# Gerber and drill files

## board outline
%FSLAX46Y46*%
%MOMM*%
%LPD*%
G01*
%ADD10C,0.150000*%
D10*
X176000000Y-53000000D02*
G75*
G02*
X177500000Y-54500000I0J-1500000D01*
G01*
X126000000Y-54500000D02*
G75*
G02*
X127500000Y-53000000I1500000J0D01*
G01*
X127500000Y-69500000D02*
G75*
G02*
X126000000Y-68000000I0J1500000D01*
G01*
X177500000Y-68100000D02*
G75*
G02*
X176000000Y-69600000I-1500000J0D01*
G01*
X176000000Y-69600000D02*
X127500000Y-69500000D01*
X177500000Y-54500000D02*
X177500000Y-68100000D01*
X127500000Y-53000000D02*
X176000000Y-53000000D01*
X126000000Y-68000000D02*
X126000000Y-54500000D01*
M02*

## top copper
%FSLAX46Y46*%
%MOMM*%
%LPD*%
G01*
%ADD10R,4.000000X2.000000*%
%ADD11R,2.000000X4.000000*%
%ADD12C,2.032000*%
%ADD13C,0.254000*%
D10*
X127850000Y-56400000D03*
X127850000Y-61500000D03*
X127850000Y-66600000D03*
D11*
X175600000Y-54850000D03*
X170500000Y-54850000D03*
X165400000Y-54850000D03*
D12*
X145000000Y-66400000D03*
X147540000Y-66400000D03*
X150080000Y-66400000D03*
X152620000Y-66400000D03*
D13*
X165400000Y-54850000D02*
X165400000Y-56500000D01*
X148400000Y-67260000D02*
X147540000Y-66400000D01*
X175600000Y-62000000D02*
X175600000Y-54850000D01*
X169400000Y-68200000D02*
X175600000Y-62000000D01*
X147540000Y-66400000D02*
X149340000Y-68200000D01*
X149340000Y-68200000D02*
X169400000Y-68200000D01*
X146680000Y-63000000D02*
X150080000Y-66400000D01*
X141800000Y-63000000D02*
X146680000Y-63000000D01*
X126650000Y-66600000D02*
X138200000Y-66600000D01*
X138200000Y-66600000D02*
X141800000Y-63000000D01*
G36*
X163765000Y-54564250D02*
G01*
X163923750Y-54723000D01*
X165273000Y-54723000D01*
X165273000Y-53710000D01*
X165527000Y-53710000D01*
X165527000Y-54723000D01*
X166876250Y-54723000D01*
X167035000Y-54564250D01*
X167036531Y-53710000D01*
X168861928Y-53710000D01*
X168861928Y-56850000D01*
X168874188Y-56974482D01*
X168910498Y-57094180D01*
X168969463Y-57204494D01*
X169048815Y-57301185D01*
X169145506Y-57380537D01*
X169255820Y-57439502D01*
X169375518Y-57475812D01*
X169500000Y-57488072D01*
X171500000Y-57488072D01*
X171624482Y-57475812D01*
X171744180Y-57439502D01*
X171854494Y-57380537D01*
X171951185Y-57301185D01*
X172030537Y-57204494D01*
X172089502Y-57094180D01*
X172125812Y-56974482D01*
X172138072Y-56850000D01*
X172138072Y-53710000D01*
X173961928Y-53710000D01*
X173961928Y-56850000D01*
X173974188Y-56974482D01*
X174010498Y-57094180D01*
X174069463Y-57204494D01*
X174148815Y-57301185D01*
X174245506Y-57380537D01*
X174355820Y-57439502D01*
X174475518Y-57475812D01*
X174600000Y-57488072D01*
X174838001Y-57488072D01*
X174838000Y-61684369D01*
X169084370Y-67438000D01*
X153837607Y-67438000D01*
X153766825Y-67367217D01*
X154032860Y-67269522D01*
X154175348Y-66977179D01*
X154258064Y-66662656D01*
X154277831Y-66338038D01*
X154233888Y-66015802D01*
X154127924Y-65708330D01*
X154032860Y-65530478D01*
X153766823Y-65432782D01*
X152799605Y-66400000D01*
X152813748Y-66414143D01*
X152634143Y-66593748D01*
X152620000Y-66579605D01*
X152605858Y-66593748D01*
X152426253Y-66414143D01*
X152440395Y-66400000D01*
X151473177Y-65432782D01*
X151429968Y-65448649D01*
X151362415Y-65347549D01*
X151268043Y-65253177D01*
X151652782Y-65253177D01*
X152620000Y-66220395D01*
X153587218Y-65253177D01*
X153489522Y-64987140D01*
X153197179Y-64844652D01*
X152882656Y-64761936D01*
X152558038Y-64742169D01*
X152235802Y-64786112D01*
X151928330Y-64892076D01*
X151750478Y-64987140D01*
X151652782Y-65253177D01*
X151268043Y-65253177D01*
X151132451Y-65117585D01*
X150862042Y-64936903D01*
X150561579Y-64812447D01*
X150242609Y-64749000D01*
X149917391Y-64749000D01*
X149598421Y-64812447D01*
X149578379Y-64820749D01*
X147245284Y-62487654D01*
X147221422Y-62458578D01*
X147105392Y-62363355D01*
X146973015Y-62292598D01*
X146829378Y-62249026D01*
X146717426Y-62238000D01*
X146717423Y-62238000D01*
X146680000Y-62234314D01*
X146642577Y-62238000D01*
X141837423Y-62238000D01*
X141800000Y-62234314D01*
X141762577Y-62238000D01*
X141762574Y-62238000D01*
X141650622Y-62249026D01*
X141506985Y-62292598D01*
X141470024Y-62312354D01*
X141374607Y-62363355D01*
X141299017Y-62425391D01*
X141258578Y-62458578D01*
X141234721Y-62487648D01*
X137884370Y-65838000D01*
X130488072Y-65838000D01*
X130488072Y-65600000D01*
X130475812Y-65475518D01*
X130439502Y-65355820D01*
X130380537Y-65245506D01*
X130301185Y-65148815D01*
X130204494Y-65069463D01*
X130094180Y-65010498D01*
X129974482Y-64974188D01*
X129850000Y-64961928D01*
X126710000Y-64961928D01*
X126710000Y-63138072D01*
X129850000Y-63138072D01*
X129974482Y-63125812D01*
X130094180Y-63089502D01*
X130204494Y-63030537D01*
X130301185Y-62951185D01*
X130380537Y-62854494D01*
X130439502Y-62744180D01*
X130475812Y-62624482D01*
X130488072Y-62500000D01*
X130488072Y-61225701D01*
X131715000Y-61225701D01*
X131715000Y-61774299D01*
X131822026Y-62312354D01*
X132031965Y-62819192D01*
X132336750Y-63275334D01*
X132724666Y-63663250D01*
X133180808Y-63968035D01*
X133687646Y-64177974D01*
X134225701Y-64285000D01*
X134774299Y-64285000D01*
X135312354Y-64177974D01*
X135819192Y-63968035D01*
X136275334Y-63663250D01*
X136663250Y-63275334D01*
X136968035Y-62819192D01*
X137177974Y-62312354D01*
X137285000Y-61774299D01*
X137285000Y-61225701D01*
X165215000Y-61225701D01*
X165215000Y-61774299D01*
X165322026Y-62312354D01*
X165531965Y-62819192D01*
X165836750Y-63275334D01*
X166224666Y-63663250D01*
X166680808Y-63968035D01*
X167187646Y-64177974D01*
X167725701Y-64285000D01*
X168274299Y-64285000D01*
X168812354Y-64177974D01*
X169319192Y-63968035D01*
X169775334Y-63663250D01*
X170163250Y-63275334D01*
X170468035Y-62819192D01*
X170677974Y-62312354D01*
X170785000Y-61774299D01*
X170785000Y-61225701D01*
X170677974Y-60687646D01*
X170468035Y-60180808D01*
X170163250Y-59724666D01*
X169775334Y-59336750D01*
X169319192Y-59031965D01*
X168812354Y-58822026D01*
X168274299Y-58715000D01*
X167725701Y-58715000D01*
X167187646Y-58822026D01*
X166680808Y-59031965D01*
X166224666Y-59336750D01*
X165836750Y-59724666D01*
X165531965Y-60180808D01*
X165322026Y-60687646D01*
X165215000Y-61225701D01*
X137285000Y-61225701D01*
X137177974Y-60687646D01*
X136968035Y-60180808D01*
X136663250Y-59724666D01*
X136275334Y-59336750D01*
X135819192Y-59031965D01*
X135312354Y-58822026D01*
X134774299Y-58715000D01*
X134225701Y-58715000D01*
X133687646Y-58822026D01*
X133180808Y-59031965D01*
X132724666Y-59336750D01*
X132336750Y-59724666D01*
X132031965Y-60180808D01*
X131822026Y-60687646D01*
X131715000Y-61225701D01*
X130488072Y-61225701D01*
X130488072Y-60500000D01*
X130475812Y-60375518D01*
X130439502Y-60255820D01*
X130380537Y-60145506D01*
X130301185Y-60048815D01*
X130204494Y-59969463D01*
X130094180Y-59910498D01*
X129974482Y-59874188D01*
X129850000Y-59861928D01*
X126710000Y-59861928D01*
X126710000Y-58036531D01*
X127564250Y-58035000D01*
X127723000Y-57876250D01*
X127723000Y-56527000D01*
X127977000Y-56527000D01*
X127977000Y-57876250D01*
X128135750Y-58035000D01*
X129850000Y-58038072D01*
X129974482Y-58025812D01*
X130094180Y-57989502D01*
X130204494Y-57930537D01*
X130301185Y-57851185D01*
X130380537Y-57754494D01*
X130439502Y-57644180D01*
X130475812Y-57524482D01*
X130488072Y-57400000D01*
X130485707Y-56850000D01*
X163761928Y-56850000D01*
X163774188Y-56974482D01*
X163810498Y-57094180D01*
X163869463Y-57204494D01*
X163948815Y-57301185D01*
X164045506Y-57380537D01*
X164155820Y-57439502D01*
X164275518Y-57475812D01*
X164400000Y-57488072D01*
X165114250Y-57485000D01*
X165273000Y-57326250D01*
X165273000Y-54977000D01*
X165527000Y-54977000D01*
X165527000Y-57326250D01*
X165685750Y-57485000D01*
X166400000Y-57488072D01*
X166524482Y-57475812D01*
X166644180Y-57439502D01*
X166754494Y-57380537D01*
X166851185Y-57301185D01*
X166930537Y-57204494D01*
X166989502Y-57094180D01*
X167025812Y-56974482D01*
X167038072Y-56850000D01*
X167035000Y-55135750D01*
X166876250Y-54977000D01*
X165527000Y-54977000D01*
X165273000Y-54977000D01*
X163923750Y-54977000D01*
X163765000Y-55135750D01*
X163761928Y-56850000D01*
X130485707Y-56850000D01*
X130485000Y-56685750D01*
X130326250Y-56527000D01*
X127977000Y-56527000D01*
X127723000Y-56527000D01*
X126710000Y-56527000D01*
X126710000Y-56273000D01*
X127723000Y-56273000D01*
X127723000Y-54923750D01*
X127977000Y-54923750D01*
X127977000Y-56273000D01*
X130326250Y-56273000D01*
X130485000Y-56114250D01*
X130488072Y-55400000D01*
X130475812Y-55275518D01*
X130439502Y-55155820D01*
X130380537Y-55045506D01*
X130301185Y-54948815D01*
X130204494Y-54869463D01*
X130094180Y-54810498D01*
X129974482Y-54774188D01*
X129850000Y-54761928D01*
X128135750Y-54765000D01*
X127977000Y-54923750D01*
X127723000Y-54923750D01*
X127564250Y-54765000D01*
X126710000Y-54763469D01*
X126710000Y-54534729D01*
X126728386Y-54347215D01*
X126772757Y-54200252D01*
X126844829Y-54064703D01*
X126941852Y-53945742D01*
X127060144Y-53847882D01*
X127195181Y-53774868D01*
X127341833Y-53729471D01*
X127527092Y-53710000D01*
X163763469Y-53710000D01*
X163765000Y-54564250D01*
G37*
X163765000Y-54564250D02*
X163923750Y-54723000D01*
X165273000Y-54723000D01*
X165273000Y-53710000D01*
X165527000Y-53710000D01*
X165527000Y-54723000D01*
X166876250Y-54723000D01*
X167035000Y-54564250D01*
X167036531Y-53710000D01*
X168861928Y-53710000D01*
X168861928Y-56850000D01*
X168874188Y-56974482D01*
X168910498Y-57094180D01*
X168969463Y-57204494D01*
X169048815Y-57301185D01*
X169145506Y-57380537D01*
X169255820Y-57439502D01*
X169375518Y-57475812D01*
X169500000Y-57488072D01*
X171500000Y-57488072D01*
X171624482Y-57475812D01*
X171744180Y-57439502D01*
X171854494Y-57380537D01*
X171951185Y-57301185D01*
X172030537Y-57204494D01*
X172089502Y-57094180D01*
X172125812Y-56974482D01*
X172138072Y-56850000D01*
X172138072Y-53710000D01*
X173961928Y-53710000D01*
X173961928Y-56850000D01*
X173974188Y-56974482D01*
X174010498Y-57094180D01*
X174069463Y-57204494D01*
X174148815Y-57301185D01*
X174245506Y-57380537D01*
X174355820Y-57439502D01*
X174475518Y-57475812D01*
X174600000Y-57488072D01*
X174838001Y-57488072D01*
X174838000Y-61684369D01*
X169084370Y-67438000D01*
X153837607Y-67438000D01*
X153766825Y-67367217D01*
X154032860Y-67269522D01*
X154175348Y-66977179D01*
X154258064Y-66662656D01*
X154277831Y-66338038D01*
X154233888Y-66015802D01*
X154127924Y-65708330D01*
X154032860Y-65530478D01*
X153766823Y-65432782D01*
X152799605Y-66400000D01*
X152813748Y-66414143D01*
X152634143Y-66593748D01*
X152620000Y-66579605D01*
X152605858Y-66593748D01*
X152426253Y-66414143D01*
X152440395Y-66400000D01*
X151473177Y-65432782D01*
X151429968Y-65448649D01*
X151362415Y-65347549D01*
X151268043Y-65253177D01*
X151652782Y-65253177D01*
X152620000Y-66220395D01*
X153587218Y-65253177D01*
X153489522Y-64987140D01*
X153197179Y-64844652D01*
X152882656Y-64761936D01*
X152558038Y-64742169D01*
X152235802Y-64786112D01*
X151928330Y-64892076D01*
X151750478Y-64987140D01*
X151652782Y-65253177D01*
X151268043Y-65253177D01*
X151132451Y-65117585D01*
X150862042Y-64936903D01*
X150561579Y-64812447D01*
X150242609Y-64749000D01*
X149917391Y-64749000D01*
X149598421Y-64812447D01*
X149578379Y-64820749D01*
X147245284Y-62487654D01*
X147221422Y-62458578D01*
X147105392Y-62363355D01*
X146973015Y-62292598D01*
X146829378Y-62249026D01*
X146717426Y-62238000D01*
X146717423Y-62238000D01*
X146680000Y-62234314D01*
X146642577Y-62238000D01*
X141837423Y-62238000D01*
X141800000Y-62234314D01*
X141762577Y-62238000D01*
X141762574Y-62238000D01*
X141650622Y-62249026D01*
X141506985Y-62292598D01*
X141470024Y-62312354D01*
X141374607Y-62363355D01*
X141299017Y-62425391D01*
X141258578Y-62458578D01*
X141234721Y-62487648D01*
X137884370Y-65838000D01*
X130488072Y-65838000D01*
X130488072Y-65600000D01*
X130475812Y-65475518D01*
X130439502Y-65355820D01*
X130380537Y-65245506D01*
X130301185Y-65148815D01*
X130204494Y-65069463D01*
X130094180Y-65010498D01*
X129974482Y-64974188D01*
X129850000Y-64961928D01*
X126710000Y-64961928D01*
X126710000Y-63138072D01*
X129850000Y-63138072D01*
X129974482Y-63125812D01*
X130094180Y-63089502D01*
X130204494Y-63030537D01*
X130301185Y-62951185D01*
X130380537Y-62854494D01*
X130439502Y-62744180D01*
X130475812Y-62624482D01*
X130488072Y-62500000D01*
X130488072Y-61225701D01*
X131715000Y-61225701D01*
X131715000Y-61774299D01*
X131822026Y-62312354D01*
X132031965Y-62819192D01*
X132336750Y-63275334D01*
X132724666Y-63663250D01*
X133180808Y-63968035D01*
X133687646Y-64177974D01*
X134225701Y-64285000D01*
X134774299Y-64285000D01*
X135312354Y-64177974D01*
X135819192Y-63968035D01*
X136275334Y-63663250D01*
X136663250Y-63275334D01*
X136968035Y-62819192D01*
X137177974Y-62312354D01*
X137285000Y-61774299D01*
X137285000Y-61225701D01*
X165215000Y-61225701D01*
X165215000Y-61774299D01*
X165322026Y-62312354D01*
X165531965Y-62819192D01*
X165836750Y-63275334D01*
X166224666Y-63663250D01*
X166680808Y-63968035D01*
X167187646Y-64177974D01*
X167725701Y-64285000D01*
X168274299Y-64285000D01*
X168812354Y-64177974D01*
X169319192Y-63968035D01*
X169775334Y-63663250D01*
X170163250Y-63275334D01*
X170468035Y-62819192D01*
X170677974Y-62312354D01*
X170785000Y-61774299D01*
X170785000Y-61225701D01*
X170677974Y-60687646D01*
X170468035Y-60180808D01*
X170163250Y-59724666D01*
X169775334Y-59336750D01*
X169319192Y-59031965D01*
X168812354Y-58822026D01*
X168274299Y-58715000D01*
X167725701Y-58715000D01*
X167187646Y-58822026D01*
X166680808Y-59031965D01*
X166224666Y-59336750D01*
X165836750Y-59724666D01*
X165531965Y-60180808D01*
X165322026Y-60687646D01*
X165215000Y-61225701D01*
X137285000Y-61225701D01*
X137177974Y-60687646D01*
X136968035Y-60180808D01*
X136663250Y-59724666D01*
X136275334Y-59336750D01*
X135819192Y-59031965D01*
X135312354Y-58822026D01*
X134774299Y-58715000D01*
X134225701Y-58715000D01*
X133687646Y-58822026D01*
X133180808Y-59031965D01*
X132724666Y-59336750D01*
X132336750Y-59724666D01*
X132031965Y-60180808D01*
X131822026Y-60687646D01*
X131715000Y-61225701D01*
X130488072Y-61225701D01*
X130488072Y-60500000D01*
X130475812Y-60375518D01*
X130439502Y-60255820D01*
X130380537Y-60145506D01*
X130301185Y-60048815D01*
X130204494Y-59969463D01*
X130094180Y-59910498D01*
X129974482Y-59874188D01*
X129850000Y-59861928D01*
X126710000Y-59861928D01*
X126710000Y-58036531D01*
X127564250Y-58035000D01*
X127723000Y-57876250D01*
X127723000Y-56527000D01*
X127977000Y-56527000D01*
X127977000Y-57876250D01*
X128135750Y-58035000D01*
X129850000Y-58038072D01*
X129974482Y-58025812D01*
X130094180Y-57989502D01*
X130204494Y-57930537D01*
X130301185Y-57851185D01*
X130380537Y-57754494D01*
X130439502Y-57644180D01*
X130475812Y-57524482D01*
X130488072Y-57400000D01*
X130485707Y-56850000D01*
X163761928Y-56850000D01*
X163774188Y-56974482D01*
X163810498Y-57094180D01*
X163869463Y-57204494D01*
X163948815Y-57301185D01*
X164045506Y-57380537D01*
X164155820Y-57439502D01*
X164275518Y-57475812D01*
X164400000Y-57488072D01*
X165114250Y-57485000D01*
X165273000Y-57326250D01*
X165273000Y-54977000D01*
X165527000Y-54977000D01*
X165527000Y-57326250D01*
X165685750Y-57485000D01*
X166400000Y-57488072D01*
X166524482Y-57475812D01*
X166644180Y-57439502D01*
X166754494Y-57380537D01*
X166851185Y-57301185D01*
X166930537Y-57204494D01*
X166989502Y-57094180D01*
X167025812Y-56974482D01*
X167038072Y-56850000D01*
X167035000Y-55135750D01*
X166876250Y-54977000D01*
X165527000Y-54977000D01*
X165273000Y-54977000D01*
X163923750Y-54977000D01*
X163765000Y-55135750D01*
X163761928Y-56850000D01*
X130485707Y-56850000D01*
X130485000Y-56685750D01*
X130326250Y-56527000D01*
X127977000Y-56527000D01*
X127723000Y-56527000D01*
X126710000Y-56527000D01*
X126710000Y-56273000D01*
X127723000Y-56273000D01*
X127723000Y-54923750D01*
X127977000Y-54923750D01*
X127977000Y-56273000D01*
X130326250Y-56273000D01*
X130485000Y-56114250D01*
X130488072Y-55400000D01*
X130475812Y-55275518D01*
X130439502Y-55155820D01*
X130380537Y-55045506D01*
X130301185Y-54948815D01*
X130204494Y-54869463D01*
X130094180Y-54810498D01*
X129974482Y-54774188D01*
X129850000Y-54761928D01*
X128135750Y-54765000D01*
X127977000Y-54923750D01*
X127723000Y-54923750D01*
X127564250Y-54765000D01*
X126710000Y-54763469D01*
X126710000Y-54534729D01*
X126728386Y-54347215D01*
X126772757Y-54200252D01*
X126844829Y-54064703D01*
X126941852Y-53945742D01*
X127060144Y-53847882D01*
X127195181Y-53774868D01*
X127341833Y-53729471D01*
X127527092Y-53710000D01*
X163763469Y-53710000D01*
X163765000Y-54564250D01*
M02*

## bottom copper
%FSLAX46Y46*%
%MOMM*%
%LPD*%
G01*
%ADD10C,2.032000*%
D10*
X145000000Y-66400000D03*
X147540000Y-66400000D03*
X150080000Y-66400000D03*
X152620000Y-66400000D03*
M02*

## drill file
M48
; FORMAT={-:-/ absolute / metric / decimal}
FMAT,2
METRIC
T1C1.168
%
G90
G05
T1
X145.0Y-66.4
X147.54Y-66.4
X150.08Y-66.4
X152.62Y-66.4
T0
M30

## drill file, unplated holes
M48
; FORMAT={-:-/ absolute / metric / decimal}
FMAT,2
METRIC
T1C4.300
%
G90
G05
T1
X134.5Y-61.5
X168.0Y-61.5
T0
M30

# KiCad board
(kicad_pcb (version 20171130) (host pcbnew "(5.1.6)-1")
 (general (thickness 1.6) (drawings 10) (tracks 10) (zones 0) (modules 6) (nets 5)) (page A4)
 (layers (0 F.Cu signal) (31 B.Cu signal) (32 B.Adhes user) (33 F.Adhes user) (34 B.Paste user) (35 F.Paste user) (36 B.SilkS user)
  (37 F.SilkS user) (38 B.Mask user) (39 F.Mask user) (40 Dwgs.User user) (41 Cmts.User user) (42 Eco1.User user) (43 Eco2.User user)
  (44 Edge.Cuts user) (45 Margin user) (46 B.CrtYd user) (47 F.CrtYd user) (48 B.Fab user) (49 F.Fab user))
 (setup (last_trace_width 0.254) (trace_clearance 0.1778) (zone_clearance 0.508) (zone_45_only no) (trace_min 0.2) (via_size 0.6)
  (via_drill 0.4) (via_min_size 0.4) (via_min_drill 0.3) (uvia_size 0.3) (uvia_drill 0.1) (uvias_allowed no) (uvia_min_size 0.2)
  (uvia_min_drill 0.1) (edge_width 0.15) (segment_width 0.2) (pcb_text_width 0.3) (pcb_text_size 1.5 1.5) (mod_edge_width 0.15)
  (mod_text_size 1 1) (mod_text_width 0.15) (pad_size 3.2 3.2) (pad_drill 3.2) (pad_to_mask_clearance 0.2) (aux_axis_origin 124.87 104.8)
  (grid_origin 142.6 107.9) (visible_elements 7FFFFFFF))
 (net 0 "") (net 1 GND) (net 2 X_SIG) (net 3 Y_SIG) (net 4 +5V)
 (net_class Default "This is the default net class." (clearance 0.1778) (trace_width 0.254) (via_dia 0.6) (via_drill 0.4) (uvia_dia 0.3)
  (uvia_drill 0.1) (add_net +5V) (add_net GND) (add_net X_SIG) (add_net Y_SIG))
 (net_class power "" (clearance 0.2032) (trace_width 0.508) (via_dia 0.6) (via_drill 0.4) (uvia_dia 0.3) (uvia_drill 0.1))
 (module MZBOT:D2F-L (layer F.Cu) (at 119.25 67.9 90)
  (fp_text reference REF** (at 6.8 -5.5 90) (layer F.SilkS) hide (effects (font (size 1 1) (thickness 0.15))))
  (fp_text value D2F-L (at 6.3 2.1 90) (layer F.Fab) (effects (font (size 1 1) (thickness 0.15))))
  (pad 3 connect rect (at 11.5 8.6 90) (size 2 4) (layers F.Cu F.Mask) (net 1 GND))
  (pad 2 connect rect (at 6.4 8.6 90) (size 2 4) (layers F.Cu F.Mask))
  (pad 1 connect rect (at 1.3 8.6 90) (size 2 4) (layers F.Cu F.Mask) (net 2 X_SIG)))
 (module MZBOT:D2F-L (layer F.Cu) (at 164.1 46.25)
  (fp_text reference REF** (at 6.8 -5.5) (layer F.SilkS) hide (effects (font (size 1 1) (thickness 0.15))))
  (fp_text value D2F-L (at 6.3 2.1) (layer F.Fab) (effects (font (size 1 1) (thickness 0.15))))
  (pad 3 connect rect (at 11.5 8.6) (size 2 4) (layers F.Cu F.Mask) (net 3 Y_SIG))
  (pad 2 connect rect (at 6.4 8.6) (size 2 4) (layers F.Cu F.Mask))
  (pad 1 connect rect (at 1.3 8.6) (size 2 4) (layers F.Cu F.Mask) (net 1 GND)))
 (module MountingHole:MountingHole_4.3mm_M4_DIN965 (layer F.Cu) (at 168 61.5)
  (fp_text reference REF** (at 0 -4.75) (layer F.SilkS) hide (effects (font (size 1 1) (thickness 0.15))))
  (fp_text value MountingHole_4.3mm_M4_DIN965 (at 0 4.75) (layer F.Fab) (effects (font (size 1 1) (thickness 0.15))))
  (pad 1 np_thru_hole circle (at 0 0) (size 4.3 4.3) (drill 4.3) (layers *.Cu *.Mask)))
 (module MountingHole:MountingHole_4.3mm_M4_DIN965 (layer F.Cu) (at 134.5 61.5)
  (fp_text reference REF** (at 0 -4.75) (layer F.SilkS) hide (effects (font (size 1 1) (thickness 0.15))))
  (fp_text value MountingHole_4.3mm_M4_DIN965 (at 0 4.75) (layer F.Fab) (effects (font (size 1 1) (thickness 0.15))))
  (pad 1 np_thru_hole circle (at 0 0) (size 4.3 4.3) (drill 4.3) (layers *.Cu *.Mask)))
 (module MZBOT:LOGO (layer F.Cu) (at 152.25 61.5)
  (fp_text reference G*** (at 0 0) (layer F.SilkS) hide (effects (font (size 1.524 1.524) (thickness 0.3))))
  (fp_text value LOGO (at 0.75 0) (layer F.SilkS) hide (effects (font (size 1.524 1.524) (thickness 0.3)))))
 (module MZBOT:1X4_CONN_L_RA (layer B.Cu) (at 148.81 66.4 90)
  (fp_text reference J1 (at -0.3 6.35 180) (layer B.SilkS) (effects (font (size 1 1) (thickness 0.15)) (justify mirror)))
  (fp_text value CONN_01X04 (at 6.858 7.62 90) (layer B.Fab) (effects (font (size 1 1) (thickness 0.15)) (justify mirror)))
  (pad 4 thru_hole circle (at 0 -3.81 90) (size 2.032 2.032) (drill 1.1684) (layers *.Cu *.Mask B.SilkS) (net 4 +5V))
  (pad 3 thru_hole circle (at 0 -1.27 90) (size 2.032 2.032) (drill 1.1684) (layers *.Cu *.Mask B.SilkS) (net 3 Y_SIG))
  (pad 2 thru_hole circle (at 0 1.27 90) (size 2.032 2.032) (drill 1.1684) (layers *.Cu *.Mask B.SilkS) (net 2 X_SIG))
  (pad 1 thru_hole circle (at 0 3.81 90) (size 2.032 2.032) (drill 1.1684) (layers *.Cu *.Mask B.SilkS) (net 1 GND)))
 (gr_arc (start 176 54.5) (end 177.5 54.5) (angle -90) (layer Edge.Cuts) (width 0.15))
 (gr_arc (start 127.5 54.5) (end 127.5 53) (angle -90) (layer Edge.Cuts) (width 0.15))
 (gr_arc (start 127.5 68) (end 126 68) (angle -90) (layer Edge.Cuts) (width 0.15))
 (gr_arc (start 176 68.1) (end 176 69.6) (angle -90) (layer Edge.Cuts) (width 0.15))
 (gr_line (start 176 69.6) (end 127.5 69.5) (layer Edge.Cuts) (width 0.15))
 (gr_line (start 177.5 54.5) (end 177.5 68.1) (layer Edge.Cuts) (width 0.15))
 (gr_line (start 127.5 53) (end 176 53) (layer Edge.Cuts) (width 0.15))
 (gr_line (start 126 68) (end 126 54.5) (layer Edge.Cuts) (width 0.15))
 (segment (start 165.4 54.85) (end 165.4 56.5) (width 0.254) (layer F.Cu) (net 1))
 (segment (start 148.4 67.26) (end 147.54 66.4) (width 0.254) (layer F.Cu) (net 3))
 (segment (start 175.6 62) (end 175.6 54.85) (width 0.254) (layer F.Cu) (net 3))
 (segment (start 169.4 68.2) (end 175.6 62) (width 0.254) (layer F.Cu) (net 3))
 (segment (start 147.54 66.4) (end 149.34 68.2) (width 0.254) (layer F.Cu) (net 3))
 (segment (start 149.34 68.2) (end 169.4 68.2) (width 0.254) (layer F.Cu) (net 3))
 (segment (start 146.68 63) (end 150.08 66.4) (width 0.254) (layer F.Cu) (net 2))
 (segment (start 141.8 63) (end 146.68 63) (width 0.254) (layer F.Cu) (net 2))
 (segment (start 126.65 66.6) (end 138.2 66.6) (width 0.254) (layer F.Cu) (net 2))
 (segment (start 138.2 66.6) (end 141.8 63) (width 0.254) (layer F.Cu) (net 2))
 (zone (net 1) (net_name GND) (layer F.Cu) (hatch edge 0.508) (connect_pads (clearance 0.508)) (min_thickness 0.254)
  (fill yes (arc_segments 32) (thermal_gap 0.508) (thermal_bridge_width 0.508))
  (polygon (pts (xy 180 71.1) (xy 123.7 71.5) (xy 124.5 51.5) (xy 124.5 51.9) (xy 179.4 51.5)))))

